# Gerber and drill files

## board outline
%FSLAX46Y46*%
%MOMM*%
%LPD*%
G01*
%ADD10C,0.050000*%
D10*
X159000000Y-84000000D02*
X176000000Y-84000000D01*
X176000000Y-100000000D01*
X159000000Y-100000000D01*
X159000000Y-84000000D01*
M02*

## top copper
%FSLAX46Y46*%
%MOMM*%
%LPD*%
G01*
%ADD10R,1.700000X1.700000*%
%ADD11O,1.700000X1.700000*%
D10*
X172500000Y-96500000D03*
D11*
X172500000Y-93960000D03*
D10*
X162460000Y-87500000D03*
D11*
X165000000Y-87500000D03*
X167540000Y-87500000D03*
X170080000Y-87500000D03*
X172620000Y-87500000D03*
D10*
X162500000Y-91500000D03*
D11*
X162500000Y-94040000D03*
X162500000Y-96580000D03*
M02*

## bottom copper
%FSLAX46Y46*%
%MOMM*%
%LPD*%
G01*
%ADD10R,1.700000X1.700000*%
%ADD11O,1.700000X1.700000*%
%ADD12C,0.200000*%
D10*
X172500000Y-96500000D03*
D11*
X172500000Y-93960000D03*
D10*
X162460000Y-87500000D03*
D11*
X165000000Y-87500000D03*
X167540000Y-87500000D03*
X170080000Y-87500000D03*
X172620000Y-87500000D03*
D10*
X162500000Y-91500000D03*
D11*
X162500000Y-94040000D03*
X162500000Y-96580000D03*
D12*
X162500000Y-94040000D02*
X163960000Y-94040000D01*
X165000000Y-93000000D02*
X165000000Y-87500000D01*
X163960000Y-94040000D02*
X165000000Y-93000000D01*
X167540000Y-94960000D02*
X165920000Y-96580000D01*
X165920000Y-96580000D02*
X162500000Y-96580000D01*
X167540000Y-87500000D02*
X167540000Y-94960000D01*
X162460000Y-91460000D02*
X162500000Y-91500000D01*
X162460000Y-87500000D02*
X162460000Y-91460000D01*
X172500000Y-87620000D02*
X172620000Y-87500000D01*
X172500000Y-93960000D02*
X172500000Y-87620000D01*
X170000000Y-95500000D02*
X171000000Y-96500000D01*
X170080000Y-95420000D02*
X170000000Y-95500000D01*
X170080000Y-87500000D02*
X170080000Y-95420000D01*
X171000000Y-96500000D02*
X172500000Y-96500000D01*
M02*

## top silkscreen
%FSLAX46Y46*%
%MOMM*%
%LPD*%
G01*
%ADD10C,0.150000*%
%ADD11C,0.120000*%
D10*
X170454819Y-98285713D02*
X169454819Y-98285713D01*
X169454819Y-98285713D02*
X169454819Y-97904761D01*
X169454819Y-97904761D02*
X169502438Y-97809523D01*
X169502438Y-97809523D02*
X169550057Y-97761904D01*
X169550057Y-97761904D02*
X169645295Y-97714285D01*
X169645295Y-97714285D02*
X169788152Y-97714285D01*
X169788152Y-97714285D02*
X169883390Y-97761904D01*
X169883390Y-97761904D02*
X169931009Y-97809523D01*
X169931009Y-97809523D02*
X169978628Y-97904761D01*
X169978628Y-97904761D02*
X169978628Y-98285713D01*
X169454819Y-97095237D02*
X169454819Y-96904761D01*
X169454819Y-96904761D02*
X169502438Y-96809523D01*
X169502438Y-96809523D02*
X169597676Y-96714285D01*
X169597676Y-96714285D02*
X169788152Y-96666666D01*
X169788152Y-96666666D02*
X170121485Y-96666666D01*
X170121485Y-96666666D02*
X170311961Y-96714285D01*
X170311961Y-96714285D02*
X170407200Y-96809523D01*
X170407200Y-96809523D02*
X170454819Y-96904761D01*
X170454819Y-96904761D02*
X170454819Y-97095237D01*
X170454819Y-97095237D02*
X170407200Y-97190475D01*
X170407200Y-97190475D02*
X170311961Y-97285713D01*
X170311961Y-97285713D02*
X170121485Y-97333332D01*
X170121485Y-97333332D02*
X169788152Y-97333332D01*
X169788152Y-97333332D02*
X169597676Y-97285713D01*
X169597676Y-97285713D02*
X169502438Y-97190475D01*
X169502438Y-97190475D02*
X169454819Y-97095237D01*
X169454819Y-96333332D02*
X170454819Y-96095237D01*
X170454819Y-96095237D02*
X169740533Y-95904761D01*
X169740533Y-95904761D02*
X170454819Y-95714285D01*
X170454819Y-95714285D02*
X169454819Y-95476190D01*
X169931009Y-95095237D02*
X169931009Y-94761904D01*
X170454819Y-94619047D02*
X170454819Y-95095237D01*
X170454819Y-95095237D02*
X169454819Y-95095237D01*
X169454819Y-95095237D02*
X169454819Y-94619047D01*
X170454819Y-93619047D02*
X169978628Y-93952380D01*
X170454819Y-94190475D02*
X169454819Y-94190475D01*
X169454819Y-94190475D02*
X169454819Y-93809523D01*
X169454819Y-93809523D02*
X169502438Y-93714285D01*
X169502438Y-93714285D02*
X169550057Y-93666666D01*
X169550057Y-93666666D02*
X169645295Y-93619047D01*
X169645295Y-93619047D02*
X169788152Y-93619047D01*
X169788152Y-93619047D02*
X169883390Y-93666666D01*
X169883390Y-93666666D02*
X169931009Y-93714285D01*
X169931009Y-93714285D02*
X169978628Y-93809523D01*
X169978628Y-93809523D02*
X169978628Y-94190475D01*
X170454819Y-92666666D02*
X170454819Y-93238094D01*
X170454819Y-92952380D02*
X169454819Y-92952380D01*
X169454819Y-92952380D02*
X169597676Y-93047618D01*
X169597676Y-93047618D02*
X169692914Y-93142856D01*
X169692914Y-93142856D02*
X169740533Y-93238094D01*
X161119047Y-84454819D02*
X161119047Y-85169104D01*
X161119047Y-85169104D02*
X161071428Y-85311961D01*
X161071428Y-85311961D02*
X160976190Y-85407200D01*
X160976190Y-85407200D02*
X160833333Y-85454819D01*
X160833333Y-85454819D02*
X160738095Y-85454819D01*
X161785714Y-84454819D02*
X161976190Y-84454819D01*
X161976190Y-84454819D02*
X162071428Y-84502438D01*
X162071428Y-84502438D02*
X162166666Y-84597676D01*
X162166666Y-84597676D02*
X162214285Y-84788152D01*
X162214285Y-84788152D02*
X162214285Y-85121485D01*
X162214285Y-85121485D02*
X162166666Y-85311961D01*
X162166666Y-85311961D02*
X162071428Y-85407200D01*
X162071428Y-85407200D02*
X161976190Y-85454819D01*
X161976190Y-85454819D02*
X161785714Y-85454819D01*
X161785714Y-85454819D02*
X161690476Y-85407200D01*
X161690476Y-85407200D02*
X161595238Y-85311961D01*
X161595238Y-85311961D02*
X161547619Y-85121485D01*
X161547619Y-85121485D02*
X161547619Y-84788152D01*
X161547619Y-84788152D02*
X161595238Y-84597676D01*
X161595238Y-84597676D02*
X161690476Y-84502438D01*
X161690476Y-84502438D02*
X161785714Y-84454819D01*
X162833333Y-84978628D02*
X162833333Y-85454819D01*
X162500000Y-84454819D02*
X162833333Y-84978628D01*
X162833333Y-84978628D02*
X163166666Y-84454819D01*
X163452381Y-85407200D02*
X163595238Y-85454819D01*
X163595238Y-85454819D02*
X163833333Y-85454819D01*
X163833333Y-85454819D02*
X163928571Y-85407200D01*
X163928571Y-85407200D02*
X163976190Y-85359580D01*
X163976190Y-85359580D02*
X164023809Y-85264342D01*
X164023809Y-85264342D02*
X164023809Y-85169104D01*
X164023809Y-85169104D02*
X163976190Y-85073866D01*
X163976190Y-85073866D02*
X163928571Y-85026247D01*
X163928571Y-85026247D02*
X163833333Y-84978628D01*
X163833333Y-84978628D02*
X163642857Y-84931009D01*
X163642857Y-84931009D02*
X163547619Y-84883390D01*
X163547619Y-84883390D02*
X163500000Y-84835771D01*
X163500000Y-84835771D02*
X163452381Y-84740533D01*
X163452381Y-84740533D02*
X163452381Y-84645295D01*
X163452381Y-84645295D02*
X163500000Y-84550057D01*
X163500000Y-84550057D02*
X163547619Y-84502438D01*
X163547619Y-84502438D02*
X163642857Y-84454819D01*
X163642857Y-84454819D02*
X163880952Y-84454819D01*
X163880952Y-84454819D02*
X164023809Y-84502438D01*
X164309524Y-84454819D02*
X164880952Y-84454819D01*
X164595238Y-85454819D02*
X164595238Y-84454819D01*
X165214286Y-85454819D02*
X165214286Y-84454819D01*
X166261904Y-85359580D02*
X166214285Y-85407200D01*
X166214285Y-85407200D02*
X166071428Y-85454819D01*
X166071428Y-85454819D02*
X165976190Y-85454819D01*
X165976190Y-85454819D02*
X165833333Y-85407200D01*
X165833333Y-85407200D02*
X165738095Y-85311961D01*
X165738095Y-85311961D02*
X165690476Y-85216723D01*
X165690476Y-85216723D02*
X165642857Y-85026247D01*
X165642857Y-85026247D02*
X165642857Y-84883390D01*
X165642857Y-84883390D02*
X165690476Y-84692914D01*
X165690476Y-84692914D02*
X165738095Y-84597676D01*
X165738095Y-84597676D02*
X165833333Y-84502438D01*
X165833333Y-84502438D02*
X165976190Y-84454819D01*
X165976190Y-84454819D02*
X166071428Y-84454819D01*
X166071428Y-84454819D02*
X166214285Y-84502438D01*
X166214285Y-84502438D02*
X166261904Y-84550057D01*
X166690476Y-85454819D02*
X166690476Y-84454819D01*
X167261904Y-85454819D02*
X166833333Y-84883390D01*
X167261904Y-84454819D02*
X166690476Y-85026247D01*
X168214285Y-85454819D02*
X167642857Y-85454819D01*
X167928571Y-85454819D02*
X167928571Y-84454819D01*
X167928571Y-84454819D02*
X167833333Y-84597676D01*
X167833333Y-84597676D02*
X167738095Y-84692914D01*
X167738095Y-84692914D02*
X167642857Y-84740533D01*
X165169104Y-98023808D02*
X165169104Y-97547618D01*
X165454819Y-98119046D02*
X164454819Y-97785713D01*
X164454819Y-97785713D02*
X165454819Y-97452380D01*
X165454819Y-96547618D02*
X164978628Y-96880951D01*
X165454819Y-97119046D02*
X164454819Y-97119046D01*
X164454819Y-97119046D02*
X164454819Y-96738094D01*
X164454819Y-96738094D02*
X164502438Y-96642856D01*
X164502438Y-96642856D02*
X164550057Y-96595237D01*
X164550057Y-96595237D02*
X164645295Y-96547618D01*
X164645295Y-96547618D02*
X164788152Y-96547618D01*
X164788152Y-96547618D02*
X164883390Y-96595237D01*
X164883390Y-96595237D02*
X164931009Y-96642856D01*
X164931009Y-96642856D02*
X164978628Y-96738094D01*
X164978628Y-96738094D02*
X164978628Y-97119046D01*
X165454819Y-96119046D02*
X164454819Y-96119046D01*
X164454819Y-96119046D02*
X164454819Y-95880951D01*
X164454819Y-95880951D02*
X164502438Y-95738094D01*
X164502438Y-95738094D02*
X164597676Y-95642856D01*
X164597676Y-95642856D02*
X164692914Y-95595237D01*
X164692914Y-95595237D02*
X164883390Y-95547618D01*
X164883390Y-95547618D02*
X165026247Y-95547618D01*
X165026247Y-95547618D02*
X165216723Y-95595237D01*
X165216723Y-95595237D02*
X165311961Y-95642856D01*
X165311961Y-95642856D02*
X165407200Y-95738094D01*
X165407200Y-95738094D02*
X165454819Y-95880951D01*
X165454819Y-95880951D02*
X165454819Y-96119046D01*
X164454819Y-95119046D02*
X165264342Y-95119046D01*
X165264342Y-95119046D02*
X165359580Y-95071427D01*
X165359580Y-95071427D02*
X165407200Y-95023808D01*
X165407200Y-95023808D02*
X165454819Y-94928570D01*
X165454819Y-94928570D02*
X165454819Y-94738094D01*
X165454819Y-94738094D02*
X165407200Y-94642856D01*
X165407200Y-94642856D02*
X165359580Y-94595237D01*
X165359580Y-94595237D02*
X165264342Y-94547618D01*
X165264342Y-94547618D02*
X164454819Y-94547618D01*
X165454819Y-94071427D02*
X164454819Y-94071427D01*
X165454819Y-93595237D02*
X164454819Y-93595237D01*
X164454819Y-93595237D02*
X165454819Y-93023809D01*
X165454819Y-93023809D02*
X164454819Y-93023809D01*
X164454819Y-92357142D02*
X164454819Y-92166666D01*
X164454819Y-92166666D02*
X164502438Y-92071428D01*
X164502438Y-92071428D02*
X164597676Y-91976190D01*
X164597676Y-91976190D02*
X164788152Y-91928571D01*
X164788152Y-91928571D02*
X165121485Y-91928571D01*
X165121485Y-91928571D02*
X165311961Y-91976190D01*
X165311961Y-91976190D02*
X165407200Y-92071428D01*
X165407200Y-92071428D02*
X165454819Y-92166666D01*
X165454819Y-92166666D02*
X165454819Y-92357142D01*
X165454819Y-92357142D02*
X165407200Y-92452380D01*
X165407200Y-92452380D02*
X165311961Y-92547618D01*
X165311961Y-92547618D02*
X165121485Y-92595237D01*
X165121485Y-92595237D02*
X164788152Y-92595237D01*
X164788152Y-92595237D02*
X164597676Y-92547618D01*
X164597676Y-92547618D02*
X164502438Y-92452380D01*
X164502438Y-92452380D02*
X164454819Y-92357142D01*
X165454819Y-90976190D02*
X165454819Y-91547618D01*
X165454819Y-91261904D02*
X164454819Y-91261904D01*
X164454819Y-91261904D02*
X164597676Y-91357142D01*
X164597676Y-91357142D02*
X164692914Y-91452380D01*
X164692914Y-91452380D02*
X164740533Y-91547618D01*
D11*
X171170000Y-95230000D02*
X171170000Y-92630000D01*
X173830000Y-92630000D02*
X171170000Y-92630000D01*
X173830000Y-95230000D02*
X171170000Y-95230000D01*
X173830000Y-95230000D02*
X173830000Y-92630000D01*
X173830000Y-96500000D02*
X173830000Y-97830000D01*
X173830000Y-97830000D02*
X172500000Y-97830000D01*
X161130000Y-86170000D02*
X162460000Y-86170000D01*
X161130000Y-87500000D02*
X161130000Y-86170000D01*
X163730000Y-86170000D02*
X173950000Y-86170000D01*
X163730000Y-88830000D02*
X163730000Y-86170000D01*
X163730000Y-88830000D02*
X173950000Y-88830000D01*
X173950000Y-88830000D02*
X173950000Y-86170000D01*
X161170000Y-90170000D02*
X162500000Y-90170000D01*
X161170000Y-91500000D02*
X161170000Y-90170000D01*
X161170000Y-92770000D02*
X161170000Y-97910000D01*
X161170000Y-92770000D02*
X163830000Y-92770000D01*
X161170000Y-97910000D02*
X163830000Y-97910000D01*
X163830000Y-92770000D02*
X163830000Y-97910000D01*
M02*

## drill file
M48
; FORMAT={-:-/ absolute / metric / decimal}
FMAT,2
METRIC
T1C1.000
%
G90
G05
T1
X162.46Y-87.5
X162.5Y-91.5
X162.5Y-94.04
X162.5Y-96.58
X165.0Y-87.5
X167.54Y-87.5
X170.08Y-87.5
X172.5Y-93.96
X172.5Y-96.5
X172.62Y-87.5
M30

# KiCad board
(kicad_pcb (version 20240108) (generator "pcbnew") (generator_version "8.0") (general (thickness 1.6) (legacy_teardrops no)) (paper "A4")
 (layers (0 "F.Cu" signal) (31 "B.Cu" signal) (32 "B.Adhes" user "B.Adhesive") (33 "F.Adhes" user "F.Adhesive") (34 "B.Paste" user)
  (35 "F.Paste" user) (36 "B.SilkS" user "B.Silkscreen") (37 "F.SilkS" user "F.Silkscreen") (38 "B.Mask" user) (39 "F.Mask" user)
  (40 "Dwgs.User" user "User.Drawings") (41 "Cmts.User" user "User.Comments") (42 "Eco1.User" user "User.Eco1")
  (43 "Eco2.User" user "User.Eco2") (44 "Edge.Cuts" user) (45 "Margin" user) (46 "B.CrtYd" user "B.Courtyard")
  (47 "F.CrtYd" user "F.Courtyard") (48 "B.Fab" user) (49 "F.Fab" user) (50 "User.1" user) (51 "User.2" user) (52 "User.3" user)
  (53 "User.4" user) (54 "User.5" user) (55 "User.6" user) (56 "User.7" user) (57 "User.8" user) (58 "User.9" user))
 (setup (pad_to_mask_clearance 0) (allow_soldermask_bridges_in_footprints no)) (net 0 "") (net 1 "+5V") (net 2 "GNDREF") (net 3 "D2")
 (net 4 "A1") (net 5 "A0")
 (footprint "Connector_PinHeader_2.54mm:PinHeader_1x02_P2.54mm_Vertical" (layer "F.Cu") (at 172.5 96.5 180)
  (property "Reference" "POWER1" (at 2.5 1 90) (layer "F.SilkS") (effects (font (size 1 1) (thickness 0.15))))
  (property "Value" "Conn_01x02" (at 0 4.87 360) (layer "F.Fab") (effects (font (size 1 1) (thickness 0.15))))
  (fp_line (start 1.33 1.27) (end 1.33 3.87) (stroke (width 0.12) (type solid)) (layer "F.SilkS"))
  (fp_line (start -1.33 3.87) (end 1.33 3.87) (stroke (width 0.12) (type solid)) (layer "F.SilkS"))
  (fp_line (start -1.33 1.27) (end 1.33 1.27) (stroke (width 0.12) (type solid)) (layer "F.SilkS"))
  (fp_line (start -1.33 1.27) (end -1.33 3.87) (stroke (width 0.12) (type solid)) (layer "F.SilkS"))
  (fp_line (start -1.33 0) (end -1.33 -1.33) (stroke (width 0.12) (type solid)) (layer "F.SilkS"))
  (fp_line (start -1.33 -1.33) (end 0 -1.33) (stroke (width 0.12) (type solid)) (layer "F.SilkS"))
  (pad "1" thru_hole rect (at 0 0 180) (size 1.7 1.7) (drill 1) (layers "*.Cu" "*.Mask") (remove_unused_layers no) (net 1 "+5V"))
  (pad "2" thru_hole oval (at 0 2.54 180) (size 1.7 1.7) (drill 1) (layers "*.Cu" "*.Mask") (remove_unused_layers no) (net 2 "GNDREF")))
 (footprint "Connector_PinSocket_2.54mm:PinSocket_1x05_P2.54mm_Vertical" (layer "F.Cu") (at 162.46 87.5 90)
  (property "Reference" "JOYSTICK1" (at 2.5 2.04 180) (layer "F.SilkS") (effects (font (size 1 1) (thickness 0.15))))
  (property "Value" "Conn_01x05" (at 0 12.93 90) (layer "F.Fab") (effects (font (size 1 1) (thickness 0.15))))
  (fp_line (start 1.33 -1.33) (end 1.33 0) (stroke (width 0.12) (type solid)) (layer "F.SilkS"))
  (fp_line (start 0 -1.33) (end 1.33 -1.33) (stroke (width 0.12) (type solid)) (layer "F.SilkS"))
  (fp_line (start 1.33 1.27) (end 1.33 11.49) (stroke (width 0.12) (type solid)) (layer "F.SilkS"))
  (fp_line (start -1.33 1.27) (end 1.33 1.27) (stroke (width 0.12) (type solid)) (layer "F.SilkS"))
  (fp_line (start -1.33 1.27) (end -1.33 11.49) (stroke (width 0.12) (type solid)) (layer "F.SilkS"))
  (fp_line (start -1.33 11.49) (end 1.33 11.49) (stroke (width 0.12) (type solid)) (layer "F.SilkS"))
  (pad "1" thru_hole rect (at 0 0 90) (size 1.7 1.7) (drill 1) (layers "*.Cu" "*.Mask") (remove_unused_layers no) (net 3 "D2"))
  (pad "2" thru_hole oval (at 0 2.54 90) (size 1.7 1.7) (drill 1) (layers "*.Cu" "*.Mask") (remove_unused_layers no) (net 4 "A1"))
  (pad "3" thru_hole oval (at 0 5.08 90) (size 1.7 1.7) (drill 1) (layers "*.Cu" "*.Mask") (remove_unused_layers no) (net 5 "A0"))
  (pad "4" thru_hole oval (at 0 7.62 90) (size 1.7 1.7) (drill 1) (layers "*.Cu" "*.Mask") (remove_unused_layers no) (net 1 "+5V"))
  (pad "5" thru_hole oval (at 0 10.16 90) (size 1.7 1.7) (drill 1) (layers "*.Cu" "*.Mask") (remove_unused_layers no) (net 2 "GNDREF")))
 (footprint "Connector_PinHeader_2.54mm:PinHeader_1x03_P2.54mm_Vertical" (layer "F.Cu") (at 162.5 91.5)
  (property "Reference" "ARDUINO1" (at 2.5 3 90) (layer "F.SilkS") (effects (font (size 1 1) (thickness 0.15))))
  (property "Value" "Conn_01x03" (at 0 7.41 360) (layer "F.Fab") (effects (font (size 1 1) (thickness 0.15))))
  (fp_line (start -1.33 -1.33) (end 0 -1.33) (stroke (width 0.12) (type solid)) (layer "F.SilkS"))
  (fp_line (start -1.33 0) (end -1.33 -1.33) (stroke (width 0.12) (type solid)) (layer "F.SilkS"))
  (fp_line (start -1.33 1.27) (end -1.33 6.41) (stroke (width 0.12) (type solid)) (layer "F.SilkS"))
  (fp_line (start -1.33 1.27) (end 1.33 1.27) (stroke (width 0.12) (type solid)) (layer "F.SilkS"))
  (fp_line (start -1.33 6.41) (end 1.33 6.41) (stroke (width 0.12) (type solid)) (layer "F.SilkS"))
  (fp_line (start 1.33 1.27) (end 1.33 6.41) (stroke (width 0.12) (type solid)) (layer "F.SilkS"))
  (pad "1" thru_hole rect (at 0 0) (size 1.7 1.7) (drill 1) (layers "*.Cu" "*.Mask") (remove_unused_layers no) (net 3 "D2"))
  (pad "2" thru_hole oval (at 0 2.54) (size 1.7 1.7) (drill 1) (layers "*.Cu" "*.Mask") (remove_unused_layers no) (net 4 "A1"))
  (pad "3" thru_hole oval (at 0 5.08) (size 1.7 1.7) (drill 1) (layers "*.Cu" "*.Mask") (remove_unused_layers no) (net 5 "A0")))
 (gr_rect (start 159 84) (end 176 100) (stroke (width 0.05) (type default)) (fill none) (layer "Edge.Cuts"))
 (segment (start 162.5 94.04) (end 163.96 94.04) (width 0.2) (layer "B.Cu") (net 4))
 (segment (start 165 93) (end 165 87.5) (width 0.2) (layer "B.Cu") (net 4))
 (segment (start 163.96 94.04) (end 165 93) (width 0.2) (layer "B.Cu") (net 4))
 (segment (start 167.54 94.96) (end 165.92 96.58) (width 0.2) (layer "B.Cu") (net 5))
 (segment (start 165.92 96.58) (end 162.5 96.58) (width 0.2) (layer "B.Cu") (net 5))
 (segment (start 167.54 87.5) (end 167.54 94.96) (width 0.2) (layer "B.Cu") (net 5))
 (segment (start 162.46 91.46) (end 162.5 91.5) (width 0.2) (layer "B.Cu") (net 3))
 (segment (start 162.46 87.5) (end 162.46 91.46) (width 0.2) (layer "B.Cu") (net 3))
 (segment (start 172.5 87.62) (end 172.62 87.5) (width 0.2) (layer "B.Cu") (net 2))
 (segment (start 172.5 93.96) (end 172.5 87.62) (width 0.2) (layer "B.Cu") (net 2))
 (segment (start 170 95.5) (end 171 96.5) (width 0.2) (layer "B.Cu") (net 1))
 (segment (start 170.08 95.42) (end 170 95.5) (width 0.2) (layer "B.Cu") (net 1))
 (segment (start 170.08 87.5) (end 170.08 95.42) (width 0.2) (layer "B.Cu") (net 1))
 (segment (start 171 96.5) (end 172.5 96.5) (width 0.2) (layer "B.Cu") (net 1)))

